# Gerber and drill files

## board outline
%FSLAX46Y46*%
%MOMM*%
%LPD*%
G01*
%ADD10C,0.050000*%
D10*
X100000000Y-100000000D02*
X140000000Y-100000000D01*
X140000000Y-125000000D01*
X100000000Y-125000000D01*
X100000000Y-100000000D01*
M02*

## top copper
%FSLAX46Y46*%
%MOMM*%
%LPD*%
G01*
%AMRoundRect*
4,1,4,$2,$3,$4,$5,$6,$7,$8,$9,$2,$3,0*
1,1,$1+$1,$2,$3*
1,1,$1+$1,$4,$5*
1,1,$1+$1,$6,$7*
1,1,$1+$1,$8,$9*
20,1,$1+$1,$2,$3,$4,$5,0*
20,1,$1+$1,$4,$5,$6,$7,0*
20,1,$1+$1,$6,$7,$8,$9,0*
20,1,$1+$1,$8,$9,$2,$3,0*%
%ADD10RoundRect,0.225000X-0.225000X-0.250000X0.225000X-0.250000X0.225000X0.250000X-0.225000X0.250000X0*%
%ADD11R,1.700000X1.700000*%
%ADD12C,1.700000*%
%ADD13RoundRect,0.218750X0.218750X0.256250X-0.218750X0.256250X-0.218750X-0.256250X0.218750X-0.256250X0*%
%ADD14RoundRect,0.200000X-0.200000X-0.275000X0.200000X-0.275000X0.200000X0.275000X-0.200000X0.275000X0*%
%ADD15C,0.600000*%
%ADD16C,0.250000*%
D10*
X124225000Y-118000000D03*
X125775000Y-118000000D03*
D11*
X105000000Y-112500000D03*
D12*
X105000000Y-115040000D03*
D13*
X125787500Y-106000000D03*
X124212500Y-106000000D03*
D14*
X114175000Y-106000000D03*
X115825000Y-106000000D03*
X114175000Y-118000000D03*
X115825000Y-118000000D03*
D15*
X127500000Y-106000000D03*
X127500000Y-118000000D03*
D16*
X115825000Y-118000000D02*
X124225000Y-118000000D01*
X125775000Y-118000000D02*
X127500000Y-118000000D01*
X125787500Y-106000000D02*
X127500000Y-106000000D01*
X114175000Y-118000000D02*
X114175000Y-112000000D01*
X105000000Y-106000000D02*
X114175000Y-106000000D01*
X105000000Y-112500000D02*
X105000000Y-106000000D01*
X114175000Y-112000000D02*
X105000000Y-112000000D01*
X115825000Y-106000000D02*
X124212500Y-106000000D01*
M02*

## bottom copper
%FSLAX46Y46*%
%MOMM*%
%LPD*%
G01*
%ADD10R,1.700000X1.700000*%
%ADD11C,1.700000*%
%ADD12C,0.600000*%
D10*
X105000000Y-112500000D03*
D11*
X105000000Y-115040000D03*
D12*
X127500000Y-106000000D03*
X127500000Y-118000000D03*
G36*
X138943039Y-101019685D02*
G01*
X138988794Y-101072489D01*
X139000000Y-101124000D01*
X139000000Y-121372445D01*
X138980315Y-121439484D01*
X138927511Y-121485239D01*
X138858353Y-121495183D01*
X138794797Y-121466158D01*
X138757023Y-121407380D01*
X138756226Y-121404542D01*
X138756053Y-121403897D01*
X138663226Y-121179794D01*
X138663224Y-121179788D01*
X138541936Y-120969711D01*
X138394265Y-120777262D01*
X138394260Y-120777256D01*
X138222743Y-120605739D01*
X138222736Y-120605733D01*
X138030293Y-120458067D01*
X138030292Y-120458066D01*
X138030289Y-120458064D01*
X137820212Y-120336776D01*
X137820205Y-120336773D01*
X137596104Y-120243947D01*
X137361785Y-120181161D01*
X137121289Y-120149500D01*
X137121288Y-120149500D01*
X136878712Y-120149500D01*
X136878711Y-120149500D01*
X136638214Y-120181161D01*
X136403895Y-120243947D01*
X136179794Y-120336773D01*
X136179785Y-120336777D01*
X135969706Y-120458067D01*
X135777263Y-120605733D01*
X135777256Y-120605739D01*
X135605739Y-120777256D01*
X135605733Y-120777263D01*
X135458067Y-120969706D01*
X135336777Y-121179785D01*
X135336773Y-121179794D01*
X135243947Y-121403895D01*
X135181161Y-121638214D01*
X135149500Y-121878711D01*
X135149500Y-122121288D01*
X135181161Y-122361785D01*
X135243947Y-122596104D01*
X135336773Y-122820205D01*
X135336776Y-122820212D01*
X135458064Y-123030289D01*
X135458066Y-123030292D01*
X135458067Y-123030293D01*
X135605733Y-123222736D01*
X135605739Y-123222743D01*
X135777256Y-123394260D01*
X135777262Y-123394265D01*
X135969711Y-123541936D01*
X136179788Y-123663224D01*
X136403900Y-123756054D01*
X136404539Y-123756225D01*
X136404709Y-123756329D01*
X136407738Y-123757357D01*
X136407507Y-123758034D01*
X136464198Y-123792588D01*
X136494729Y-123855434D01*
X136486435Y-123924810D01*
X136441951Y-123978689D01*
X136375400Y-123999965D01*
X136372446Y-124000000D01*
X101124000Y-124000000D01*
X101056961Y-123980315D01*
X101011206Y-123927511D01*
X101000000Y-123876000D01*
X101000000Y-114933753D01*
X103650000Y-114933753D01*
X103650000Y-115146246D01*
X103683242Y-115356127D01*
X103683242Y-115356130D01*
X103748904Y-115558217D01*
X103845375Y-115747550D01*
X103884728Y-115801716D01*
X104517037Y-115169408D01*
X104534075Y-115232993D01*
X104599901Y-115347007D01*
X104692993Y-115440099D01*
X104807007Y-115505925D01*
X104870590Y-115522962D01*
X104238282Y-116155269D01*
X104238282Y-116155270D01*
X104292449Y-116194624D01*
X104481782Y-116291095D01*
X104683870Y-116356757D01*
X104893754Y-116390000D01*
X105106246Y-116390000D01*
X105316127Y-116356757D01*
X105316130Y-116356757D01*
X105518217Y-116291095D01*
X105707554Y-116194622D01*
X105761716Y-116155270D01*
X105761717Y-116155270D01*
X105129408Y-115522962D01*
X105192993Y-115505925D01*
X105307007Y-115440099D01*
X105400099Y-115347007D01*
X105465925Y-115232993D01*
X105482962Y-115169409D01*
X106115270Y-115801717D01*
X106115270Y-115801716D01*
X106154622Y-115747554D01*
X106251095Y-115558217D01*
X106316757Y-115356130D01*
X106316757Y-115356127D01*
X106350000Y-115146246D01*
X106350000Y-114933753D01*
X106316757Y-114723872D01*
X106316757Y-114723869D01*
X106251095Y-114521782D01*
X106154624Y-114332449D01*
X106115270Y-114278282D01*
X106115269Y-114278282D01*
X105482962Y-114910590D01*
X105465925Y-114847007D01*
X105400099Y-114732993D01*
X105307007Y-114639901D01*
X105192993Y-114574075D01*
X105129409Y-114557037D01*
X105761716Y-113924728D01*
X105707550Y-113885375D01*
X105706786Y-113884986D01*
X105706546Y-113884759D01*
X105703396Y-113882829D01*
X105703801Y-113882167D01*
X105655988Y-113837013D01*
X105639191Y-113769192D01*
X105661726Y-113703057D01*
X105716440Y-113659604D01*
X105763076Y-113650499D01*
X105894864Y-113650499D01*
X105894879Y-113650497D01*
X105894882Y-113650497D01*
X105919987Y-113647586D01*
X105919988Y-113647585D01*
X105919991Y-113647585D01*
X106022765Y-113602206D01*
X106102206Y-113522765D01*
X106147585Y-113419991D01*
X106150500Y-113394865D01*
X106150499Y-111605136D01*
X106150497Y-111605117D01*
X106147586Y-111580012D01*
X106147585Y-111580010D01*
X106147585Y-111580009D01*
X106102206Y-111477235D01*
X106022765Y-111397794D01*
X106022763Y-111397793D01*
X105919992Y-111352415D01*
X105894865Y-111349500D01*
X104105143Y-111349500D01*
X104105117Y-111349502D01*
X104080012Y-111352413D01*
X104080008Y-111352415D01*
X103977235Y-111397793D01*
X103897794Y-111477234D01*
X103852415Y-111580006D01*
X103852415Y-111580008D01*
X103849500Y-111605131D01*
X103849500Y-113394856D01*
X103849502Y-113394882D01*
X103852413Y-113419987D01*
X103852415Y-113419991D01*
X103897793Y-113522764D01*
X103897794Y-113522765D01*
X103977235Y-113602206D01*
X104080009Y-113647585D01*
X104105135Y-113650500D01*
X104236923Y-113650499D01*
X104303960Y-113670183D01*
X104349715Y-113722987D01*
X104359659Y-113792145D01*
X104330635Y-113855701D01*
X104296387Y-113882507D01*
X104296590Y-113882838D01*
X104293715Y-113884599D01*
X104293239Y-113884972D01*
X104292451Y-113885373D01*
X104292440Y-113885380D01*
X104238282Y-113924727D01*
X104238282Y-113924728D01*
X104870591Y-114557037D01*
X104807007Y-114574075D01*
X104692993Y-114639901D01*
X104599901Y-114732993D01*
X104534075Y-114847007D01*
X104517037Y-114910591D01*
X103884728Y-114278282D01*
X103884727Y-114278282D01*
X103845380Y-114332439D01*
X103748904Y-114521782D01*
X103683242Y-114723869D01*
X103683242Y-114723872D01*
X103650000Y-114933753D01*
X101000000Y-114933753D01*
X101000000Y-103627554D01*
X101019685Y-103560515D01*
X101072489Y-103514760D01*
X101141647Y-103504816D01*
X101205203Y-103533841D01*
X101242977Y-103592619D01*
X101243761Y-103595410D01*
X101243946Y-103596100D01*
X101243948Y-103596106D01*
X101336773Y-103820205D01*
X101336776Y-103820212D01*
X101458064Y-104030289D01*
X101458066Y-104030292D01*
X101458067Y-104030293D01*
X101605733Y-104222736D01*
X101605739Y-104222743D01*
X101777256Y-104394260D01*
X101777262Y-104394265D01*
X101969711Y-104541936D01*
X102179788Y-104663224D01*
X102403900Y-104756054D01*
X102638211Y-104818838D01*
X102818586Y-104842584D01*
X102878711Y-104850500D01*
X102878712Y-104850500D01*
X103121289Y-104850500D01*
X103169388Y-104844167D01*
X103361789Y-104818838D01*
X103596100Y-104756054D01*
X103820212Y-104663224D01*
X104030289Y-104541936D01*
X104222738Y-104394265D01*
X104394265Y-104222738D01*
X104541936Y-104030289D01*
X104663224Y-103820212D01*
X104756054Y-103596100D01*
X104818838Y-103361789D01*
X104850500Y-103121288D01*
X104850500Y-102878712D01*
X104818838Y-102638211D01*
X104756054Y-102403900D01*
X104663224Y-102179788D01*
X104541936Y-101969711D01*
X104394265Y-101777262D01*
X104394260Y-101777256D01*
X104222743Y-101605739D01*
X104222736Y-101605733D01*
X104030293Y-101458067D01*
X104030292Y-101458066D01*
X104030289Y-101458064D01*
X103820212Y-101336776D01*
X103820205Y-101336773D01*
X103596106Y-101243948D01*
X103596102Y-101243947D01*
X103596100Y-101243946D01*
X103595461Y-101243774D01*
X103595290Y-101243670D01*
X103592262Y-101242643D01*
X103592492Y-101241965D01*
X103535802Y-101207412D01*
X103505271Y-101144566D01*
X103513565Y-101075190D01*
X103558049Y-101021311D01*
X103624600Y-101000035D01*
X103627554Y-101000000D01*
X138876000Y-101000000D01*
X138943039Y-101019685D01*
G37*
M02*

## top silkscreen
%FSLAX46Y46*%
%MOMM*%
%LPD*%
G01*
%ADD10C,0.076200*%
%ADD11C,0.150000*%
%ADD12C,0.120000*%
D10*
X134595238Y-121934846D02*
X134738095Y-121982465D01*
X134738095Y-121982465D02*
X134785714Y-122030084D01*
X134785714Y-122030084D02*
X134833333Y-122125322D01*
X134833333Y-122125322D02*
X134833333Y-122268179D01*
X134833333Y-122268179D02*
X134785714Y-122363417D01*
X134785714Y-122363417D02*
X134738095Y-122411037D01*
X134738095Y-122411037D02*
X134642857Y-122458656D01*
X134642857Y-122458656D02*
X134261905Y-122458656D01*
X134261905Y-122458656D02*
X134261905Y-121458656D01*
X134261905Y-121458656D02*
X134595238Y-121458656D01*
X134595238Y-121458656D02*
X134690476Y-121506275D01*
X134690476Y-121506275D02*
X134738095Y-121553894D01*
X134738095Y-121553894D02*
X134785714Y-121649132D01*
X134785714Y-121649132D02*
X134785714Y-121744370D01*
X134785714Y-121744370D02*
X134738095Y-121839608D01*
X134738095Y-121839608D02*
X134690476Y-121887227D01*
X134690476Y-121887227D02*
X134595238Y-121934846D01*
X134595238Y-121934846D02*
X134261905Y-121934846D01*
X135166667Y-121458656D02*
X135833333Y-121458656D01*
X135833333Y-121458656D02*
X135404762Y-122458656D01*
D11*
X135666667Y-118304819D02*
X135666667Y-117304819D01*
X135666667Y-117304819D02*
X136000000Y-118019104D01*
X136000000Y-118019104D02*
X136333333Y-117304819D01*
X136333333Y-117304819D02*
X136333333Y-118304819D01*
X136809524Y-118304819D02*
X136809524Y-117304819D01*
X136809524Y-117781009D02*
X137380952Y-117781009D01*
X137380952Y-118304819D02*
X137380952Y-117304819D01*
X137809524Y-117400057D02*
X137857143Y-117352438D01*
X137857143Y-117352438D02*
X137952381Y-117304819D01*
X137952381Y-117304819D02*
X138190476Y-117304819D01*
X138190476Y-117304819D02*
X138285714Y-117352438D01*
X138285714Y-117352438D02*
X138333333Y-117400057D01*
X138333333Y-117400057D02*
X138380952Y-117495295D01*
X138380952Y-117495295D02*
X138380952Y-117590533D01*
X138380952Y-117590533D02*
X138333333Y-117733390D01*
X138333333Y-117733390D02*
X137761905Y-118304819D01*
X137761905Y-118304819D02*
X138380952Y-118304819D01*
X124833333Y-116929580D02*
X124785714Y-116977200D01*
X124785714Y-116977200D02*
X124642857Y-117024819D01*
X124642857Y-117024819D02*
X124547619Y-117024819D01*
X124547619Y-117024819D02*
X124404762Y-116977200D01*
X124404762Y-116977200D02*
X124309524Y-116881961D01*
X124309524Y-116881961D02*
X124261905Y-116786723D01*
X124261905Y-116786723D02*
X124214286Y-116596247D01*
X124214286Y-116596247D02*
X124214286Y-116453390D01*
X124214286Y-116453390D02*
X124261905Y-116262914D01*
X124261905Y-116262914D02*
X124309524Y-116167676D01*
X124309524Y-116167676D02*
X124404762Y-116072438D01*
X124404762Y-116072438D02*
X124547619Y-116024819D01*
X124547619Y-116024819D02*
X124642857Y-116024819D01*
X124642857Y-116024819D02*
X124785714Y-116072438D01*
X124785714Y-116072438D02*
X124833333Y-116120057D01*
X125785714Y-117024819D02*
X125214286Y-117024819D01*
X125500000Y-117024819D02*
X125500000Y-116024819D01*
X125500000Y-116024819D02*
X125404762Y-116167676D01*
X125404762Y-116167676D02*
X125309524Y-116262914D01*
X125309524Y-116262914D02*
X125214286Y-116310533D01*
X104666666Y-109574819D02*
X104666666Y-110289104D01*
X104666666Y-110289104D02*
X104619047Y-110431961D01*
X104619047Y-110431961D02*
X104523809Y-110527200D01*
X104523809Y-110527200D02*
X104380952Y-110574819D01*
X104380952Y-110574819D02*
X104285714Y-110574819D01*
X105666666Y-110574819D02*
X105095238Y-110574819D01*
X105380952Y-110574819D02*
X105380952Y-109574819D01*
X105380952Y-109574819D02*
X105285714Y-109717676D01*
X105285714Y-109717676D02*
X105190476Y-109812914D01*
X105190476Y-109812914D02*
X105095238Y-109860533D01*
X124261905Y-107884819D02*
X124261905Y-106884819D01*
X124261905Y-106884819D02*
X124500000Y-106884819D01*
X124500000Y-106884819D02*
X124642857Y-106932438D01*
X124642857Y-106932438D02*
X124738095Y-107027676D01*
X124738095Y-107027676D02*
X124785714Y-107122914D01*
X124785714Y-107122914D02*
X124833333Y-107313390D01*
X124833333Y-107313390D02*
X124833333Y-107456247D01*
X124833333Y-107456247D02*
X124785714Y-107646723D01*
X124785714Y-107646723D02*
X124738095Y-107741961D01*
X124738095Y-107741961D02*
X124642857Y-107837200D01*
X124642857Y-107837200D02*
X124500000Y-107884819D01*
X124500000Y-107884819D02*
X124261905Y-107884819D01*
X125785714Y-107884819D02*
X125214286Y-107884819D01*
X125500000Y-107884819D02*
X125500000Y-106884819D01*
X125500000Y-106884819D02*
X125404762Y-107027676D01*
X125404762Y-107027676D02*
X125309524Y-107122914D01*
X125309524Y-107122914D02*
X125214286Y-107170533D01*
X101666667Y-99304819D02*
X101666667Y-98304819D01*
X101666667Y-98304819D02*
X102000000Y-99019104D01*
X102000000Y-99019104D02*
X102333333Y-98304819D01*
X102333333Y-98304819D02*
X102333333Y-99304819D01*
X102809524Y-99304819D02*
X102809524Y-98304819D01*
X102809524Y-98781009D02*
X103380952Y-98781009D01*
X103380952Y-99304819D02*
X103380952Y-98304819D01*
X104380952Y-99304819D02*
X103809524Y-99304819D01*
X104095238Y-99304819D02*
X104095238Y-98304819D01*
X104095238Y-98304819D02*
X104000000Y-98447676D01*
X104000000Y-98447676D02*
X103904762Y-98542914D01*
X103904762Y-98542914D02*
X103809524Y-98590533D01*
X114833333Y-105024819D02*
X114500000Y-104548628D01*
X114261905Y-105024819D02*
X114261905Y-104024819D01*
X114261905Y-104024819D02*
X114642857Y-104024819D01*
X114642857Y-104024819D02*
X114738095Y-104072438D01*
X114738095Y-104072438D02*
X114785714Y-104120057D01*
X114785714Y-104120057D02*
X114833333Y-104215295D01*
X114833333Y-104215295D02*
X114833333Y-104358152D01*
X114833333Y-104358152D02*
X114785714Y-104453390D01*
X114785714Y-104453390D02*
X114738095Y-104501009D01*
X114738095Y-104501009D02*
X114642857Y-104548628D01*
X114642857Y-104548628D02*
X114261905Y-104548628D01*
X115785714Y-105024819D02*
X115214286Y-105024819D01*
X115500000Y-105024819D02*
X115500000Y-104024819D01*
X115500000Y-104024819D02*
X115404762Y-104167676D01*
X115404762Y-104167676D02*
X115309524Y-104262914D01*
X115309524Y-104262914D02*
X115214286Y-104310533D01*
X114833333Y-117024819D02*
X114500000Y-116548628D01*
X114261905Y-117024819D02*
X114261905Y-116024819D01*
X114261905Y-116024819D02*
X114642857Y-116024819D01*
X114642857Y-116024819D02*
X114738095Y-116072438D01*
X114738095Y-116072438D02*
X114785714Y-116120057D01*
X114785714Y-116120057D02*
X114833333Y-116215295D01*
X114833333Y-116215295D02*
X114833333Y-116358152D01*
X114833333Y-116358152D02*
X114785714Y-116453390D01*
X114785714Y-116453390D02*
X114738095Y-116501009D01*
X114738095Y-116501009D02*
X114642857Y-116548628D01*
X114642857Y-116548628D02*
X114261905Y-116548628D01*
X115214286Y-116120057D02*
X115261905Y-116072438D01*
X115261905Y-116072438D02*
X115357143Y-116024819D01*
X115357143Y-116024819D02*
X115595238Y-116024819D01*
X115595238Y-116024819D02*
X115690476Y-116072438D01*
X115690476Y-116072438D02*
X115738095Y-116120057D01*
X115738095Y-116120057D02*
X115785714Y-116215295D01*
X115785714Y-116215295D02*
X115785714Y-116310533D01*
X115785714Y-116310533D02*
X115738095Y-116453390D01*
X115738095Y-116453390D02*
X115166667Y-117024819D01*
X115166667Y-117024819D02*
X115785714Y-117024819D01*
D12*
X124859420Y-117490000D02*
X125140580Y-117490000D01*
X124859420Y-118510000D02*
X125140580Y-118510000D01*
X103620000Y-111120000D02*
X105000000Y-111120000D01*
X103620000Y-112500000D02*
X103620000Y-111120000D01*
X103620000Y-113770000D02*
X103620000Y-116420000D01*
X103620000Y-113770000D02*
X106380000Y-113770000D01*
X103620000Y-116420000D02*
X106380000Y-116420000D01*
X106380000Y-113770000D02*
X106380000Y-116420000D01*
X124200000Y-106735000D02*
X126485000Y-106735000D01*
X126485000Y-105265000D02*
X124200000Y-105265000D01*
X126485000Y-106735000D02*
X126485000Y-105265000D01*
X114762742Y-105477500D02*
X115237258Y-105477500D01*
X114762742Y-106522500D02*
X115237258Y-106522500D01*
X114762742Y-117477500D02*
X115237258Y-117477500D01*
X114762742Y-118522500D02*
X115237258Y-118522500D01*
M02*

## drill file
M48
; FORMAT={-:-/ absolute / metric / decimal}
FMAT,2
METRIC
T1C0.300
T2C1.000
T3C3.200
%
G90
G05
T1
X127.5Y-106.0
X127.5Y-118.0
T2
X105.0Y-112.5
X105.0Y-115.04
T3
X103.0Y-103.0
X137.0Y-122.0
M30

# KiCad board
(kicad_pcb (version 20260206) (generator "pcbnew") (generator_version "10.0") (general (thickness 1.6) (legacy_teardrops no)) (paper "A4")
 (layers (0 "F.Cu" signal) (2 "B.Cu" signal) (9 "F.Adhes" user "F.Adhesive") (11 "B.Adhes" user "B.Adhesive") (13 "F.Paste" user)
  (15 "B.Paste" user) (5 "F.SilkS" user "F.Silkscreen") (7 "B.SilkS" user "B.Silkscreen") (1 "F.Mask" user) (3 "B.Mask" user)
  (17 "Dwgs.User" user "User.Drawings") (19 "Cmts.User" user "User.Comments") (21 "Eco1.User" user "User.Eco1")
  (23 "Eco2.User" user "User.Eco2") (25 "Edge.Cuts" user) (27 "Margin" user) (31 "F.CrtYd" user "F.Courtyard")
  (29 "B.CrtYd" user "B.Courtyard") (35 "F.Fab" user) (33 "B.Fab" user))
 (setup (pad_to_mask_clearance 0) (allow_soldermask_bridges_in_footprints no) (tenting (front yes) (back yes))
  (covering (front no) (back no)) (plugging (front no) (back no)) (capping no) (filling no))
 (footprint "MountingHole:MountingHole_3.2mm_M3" (layer "F.Cu") (at 137 122)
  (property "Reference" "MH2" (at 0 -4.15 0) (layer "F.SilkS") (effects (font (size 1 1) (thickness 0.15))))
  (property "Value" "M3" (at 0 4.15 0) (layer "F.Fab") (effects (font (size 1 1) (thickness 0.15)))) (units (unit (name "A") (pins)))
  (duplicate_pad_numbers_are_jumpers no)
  (pad "" np_thru_hole circle (at 0 0) (size 3.2 3.2) (drill 3.2) (layers "*.Cu" "*.Mask")))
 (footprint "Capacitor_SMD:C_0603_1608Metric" (layer "F.Cu") (at 125 118)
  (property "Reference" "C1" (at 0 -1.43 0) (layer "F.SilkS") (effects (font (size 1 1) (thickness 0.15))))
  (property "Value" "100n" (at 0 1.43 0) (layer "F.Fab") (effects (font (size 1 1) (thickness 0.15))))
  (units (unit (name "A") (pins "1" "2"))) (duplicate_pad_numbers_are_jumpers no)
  (fp_line (start -0.14058 -0.51) (end 0.14058 -0.51) (stroke (width 0.12) (type solid)) (layer "F.SilkS"))
  (fp_line (start -0.14058 0.51) (end 0.14058 0.51) (stroke (width 0.12) (type solid)) (layer "F.SilkS"))
  (pad "1" smd roundrect (at -0.775 0) (size 0.9 0.95) (layers "F.Cu" "F.Mask" "F.Paste") (roundrect_rratio 0.25) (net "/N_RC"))
  (pad "2" smd roundrect (at 0.775 0) (size 0.9 0.95) (layers "F.Cu" "F.Mask" "F.Paste") (roundrect_rratio 0.25) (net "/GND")))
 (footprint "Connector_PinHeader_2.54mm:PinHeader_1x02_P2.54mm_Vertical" (layer "F.Cu") (at 105 112.5)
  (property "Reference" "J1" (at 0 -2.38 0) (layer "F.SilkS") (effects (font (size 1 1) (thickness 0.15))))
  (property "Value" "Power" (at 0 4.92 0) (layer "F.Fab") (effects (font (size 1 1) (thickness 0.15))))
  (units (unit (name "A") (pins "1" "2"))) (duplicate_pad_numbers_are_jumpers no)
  (fp_line (start -1.38 -1.38) (end 0 -1.38) (stroke (width 0.12) (type solid)) (layer "F.SilkS"))
  (fp_line (start -1.38 0) (end -1.38 -1.38) (stroke (width 0.12) (type solid)) (layer "F.SilkS"))
  (fp_line (start -1.38 1.27) (end -1.38 3.92) (stroke (width 0.12) (type solid)) (layer "F.SilkS"))
  (fp_line (start -1.38 1.27) (end 1.38 1.27) (stroke (width 0.12) (type solid)) (layer "F.SilkS"))
  (fp_line (start -1.38 3.92) (end 1.38 3.92) (stroke (width 0.12) (type solid)) (layer "F.SilkS"))
  (fp_line (start 1.38 1.27) (end 1.38 3.92) (stroke (width 0.12) (type solid)) (layer "F.SilkS"))
  (pad "1" thru_hole rect (at 0 0) (size 1.7 1.7) (drill 1) (layers "*.Cu" "*.Mask") (remove_unused_layers no) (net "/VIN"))
  (pad "2" thru_hole circle (at 0 2.54) (size 1.7 1.7) (drill 1) (layers "*.Cu" "*.Mask") (remove_unused_layers no) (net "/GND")))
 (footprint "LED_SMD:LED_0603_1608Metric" (layer "F.Cu") (at 125 106 180)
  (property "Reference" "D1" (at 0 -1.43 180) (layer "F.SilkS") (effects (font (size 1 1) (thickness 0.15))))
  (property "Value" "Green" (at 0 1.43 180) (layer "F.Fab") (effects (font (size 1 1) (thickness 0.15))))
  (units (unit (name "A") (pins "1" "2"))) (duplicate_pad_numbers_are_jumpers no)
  (fp_line (start 0.8 -0.735) (end -1.485 -0.735) (stroke (width 0.12) (type solid)) (layer "F.SilkS"))
  (fp_line (start -1.485 0.735) (end 0.8 0.735) (stroke (width 0.12) (type solid)) (layer "F.SilkS"))
  (fp_line (start -1.485 -0.735) (end -1.485 0.735) (stroke (width 0.12) (type solid)) (layer "F.SilkS"))
  (pad "1" smd roundrect (at -0.7875 0 180) (size 0.875 0.95) (layers "F.Cu" "F.Mask" "F.Paste") (roundrect_rratio 0.25) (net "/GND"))
  (pad "2" smd roundrect (at 0.7875 0 180) (size 0.875 0.95) (layers "F.Cu" "F.Mask" "F.Paste") (roundrect_rratio 0.25) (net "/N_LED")))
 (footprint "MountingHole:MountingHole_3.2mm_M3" (layer "F.Cu") (at 103 103)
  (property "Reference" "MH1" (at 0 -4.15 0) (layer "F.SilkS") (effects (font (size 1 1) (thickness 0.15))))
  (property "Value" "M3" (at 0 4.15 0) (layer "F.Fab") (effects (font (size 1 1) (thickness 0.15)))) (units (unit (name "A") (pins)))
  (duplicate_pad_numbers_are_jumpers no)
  (pad "" np_thru_hole circle (at 0 0) (size 3.2 3.2) (drill 3.2) (layers "*.Cu" "*.Mask")))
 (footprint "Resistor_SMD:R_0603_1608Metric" (layer "F.Cu") (at 115 106)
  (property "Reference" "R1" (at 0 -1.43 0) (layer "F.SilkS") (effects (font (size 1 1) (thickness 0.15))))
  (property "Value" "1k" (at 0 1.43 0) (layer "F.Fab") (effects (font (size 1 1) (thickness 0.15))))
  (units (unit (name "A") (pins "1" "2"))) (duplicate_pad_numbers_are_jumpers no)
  (fp_line (start -0.237258 -0.5225) (end 0.237258 -0.5225) (stroke (width 0.12) (type solid)) (layer "F.SilkS"))
  (fp_line (start -0.237258 0.5225) (end 0.237258 0.5225) (stroke (width 0.12) (type solid)) (layer "F.SilkS"))
  (pad "1" smd roundrect (at -0.825 0) (size 0.8 0.95) (layers "F.Cu" "F.Mask" "F.Paste") (roundrect_rratio 0.25) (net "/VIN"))
  (pad "2" smd roundrect (at 0.825 0) (size 0.8 0.95) (layers "F.Cu" "F.Mask" "F.Paste") (roundrect_rratio 0.25) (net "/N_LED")))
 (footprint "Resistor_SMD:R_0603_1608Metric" (layer "F.Cu") (at 115 118)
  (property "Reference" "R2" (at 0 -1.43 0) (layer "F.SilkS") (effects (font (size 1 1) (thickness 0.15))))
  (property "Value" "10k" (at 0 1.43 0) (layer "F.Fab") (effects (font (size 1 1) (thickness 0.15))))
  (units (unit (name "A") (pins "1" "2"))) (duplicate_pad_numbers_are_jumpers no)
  (fp_line (start -0.237258 -0.5225) (end 0.237258 -0.5225) (stroke (width 0.12) (type solid)) (layer "F.SilkS"))
  (fp_line (start -0.237258 0.5225) (end 0.237258 0.5225) (stroke (width 0.12) (type solid)) (layer "F.SilkS"))
  (pad "1" smd roundrect (at -0.825 0) (size 0.8 0.95) (layers "F.Cu" "F.Mask" "F.Paste") (roundrect_rratio 0.25) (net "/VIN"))
  (pad "2" smd roundrect (at 0.825 0) (size 0.8 0.95) (layers "F.Cu" "F.Mask" "F.Paste") (roundrect_rratio 0.25) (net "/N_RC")))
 (gr_rect (start 100 100) (end 140 125) (stroke (width 0.05) (type default)) (fill no) (layer "Edge.Cuts"))
 (segment (start 115.825 118) (end 124.225 118) (width 0.25) (layer "F.Cu") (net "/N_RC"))
 (segment (start 125.775 118) (end 127.5 118) (width 0.25) (layer "F.Cu") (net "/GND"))
 (segment (start 125.7875 106) (end 127.5 106) (width 0.25) (layer "F.Cu") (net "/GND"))
 (via (at 127.5 106) (size 0.6) (drill 0.3) (layers "F.Cu" "B.Cu") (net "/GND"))
 (via (at 127.5 118) (size 0.6) (drill 0.3) (layers "F.Cu" "B.Cu") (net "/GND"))
 (segment (start 114.175 118) (end 114.175 112) (width 0.25) (layer "F.Cu") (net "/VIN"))
 (segment (start 105 106) (end 114.175 106) (width 0.25) (layer "F.Cu") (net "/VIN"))
 (segment (start 105 112.5) (end 105 106) (width 0.25) (layer "F.Cu") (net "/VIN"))
 (segment (start 114.175 112) (end 105 112) (width 0.25) (layer "F.Cu") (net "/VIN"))
 (segment (start 115.825 106) (end 124.2125 106) (width 0.25) (layer "F.Cu") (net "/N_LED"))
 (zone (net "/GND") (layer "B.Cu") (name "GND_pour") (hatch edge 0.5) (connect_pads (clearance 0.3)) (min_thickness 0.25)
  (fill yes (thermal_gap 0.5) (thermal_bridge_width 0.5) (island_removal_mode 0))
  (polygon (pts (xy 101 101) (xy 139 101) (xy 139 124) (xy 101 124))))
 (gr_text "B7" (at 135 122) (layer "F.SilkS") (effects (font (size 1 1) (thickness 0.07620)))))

